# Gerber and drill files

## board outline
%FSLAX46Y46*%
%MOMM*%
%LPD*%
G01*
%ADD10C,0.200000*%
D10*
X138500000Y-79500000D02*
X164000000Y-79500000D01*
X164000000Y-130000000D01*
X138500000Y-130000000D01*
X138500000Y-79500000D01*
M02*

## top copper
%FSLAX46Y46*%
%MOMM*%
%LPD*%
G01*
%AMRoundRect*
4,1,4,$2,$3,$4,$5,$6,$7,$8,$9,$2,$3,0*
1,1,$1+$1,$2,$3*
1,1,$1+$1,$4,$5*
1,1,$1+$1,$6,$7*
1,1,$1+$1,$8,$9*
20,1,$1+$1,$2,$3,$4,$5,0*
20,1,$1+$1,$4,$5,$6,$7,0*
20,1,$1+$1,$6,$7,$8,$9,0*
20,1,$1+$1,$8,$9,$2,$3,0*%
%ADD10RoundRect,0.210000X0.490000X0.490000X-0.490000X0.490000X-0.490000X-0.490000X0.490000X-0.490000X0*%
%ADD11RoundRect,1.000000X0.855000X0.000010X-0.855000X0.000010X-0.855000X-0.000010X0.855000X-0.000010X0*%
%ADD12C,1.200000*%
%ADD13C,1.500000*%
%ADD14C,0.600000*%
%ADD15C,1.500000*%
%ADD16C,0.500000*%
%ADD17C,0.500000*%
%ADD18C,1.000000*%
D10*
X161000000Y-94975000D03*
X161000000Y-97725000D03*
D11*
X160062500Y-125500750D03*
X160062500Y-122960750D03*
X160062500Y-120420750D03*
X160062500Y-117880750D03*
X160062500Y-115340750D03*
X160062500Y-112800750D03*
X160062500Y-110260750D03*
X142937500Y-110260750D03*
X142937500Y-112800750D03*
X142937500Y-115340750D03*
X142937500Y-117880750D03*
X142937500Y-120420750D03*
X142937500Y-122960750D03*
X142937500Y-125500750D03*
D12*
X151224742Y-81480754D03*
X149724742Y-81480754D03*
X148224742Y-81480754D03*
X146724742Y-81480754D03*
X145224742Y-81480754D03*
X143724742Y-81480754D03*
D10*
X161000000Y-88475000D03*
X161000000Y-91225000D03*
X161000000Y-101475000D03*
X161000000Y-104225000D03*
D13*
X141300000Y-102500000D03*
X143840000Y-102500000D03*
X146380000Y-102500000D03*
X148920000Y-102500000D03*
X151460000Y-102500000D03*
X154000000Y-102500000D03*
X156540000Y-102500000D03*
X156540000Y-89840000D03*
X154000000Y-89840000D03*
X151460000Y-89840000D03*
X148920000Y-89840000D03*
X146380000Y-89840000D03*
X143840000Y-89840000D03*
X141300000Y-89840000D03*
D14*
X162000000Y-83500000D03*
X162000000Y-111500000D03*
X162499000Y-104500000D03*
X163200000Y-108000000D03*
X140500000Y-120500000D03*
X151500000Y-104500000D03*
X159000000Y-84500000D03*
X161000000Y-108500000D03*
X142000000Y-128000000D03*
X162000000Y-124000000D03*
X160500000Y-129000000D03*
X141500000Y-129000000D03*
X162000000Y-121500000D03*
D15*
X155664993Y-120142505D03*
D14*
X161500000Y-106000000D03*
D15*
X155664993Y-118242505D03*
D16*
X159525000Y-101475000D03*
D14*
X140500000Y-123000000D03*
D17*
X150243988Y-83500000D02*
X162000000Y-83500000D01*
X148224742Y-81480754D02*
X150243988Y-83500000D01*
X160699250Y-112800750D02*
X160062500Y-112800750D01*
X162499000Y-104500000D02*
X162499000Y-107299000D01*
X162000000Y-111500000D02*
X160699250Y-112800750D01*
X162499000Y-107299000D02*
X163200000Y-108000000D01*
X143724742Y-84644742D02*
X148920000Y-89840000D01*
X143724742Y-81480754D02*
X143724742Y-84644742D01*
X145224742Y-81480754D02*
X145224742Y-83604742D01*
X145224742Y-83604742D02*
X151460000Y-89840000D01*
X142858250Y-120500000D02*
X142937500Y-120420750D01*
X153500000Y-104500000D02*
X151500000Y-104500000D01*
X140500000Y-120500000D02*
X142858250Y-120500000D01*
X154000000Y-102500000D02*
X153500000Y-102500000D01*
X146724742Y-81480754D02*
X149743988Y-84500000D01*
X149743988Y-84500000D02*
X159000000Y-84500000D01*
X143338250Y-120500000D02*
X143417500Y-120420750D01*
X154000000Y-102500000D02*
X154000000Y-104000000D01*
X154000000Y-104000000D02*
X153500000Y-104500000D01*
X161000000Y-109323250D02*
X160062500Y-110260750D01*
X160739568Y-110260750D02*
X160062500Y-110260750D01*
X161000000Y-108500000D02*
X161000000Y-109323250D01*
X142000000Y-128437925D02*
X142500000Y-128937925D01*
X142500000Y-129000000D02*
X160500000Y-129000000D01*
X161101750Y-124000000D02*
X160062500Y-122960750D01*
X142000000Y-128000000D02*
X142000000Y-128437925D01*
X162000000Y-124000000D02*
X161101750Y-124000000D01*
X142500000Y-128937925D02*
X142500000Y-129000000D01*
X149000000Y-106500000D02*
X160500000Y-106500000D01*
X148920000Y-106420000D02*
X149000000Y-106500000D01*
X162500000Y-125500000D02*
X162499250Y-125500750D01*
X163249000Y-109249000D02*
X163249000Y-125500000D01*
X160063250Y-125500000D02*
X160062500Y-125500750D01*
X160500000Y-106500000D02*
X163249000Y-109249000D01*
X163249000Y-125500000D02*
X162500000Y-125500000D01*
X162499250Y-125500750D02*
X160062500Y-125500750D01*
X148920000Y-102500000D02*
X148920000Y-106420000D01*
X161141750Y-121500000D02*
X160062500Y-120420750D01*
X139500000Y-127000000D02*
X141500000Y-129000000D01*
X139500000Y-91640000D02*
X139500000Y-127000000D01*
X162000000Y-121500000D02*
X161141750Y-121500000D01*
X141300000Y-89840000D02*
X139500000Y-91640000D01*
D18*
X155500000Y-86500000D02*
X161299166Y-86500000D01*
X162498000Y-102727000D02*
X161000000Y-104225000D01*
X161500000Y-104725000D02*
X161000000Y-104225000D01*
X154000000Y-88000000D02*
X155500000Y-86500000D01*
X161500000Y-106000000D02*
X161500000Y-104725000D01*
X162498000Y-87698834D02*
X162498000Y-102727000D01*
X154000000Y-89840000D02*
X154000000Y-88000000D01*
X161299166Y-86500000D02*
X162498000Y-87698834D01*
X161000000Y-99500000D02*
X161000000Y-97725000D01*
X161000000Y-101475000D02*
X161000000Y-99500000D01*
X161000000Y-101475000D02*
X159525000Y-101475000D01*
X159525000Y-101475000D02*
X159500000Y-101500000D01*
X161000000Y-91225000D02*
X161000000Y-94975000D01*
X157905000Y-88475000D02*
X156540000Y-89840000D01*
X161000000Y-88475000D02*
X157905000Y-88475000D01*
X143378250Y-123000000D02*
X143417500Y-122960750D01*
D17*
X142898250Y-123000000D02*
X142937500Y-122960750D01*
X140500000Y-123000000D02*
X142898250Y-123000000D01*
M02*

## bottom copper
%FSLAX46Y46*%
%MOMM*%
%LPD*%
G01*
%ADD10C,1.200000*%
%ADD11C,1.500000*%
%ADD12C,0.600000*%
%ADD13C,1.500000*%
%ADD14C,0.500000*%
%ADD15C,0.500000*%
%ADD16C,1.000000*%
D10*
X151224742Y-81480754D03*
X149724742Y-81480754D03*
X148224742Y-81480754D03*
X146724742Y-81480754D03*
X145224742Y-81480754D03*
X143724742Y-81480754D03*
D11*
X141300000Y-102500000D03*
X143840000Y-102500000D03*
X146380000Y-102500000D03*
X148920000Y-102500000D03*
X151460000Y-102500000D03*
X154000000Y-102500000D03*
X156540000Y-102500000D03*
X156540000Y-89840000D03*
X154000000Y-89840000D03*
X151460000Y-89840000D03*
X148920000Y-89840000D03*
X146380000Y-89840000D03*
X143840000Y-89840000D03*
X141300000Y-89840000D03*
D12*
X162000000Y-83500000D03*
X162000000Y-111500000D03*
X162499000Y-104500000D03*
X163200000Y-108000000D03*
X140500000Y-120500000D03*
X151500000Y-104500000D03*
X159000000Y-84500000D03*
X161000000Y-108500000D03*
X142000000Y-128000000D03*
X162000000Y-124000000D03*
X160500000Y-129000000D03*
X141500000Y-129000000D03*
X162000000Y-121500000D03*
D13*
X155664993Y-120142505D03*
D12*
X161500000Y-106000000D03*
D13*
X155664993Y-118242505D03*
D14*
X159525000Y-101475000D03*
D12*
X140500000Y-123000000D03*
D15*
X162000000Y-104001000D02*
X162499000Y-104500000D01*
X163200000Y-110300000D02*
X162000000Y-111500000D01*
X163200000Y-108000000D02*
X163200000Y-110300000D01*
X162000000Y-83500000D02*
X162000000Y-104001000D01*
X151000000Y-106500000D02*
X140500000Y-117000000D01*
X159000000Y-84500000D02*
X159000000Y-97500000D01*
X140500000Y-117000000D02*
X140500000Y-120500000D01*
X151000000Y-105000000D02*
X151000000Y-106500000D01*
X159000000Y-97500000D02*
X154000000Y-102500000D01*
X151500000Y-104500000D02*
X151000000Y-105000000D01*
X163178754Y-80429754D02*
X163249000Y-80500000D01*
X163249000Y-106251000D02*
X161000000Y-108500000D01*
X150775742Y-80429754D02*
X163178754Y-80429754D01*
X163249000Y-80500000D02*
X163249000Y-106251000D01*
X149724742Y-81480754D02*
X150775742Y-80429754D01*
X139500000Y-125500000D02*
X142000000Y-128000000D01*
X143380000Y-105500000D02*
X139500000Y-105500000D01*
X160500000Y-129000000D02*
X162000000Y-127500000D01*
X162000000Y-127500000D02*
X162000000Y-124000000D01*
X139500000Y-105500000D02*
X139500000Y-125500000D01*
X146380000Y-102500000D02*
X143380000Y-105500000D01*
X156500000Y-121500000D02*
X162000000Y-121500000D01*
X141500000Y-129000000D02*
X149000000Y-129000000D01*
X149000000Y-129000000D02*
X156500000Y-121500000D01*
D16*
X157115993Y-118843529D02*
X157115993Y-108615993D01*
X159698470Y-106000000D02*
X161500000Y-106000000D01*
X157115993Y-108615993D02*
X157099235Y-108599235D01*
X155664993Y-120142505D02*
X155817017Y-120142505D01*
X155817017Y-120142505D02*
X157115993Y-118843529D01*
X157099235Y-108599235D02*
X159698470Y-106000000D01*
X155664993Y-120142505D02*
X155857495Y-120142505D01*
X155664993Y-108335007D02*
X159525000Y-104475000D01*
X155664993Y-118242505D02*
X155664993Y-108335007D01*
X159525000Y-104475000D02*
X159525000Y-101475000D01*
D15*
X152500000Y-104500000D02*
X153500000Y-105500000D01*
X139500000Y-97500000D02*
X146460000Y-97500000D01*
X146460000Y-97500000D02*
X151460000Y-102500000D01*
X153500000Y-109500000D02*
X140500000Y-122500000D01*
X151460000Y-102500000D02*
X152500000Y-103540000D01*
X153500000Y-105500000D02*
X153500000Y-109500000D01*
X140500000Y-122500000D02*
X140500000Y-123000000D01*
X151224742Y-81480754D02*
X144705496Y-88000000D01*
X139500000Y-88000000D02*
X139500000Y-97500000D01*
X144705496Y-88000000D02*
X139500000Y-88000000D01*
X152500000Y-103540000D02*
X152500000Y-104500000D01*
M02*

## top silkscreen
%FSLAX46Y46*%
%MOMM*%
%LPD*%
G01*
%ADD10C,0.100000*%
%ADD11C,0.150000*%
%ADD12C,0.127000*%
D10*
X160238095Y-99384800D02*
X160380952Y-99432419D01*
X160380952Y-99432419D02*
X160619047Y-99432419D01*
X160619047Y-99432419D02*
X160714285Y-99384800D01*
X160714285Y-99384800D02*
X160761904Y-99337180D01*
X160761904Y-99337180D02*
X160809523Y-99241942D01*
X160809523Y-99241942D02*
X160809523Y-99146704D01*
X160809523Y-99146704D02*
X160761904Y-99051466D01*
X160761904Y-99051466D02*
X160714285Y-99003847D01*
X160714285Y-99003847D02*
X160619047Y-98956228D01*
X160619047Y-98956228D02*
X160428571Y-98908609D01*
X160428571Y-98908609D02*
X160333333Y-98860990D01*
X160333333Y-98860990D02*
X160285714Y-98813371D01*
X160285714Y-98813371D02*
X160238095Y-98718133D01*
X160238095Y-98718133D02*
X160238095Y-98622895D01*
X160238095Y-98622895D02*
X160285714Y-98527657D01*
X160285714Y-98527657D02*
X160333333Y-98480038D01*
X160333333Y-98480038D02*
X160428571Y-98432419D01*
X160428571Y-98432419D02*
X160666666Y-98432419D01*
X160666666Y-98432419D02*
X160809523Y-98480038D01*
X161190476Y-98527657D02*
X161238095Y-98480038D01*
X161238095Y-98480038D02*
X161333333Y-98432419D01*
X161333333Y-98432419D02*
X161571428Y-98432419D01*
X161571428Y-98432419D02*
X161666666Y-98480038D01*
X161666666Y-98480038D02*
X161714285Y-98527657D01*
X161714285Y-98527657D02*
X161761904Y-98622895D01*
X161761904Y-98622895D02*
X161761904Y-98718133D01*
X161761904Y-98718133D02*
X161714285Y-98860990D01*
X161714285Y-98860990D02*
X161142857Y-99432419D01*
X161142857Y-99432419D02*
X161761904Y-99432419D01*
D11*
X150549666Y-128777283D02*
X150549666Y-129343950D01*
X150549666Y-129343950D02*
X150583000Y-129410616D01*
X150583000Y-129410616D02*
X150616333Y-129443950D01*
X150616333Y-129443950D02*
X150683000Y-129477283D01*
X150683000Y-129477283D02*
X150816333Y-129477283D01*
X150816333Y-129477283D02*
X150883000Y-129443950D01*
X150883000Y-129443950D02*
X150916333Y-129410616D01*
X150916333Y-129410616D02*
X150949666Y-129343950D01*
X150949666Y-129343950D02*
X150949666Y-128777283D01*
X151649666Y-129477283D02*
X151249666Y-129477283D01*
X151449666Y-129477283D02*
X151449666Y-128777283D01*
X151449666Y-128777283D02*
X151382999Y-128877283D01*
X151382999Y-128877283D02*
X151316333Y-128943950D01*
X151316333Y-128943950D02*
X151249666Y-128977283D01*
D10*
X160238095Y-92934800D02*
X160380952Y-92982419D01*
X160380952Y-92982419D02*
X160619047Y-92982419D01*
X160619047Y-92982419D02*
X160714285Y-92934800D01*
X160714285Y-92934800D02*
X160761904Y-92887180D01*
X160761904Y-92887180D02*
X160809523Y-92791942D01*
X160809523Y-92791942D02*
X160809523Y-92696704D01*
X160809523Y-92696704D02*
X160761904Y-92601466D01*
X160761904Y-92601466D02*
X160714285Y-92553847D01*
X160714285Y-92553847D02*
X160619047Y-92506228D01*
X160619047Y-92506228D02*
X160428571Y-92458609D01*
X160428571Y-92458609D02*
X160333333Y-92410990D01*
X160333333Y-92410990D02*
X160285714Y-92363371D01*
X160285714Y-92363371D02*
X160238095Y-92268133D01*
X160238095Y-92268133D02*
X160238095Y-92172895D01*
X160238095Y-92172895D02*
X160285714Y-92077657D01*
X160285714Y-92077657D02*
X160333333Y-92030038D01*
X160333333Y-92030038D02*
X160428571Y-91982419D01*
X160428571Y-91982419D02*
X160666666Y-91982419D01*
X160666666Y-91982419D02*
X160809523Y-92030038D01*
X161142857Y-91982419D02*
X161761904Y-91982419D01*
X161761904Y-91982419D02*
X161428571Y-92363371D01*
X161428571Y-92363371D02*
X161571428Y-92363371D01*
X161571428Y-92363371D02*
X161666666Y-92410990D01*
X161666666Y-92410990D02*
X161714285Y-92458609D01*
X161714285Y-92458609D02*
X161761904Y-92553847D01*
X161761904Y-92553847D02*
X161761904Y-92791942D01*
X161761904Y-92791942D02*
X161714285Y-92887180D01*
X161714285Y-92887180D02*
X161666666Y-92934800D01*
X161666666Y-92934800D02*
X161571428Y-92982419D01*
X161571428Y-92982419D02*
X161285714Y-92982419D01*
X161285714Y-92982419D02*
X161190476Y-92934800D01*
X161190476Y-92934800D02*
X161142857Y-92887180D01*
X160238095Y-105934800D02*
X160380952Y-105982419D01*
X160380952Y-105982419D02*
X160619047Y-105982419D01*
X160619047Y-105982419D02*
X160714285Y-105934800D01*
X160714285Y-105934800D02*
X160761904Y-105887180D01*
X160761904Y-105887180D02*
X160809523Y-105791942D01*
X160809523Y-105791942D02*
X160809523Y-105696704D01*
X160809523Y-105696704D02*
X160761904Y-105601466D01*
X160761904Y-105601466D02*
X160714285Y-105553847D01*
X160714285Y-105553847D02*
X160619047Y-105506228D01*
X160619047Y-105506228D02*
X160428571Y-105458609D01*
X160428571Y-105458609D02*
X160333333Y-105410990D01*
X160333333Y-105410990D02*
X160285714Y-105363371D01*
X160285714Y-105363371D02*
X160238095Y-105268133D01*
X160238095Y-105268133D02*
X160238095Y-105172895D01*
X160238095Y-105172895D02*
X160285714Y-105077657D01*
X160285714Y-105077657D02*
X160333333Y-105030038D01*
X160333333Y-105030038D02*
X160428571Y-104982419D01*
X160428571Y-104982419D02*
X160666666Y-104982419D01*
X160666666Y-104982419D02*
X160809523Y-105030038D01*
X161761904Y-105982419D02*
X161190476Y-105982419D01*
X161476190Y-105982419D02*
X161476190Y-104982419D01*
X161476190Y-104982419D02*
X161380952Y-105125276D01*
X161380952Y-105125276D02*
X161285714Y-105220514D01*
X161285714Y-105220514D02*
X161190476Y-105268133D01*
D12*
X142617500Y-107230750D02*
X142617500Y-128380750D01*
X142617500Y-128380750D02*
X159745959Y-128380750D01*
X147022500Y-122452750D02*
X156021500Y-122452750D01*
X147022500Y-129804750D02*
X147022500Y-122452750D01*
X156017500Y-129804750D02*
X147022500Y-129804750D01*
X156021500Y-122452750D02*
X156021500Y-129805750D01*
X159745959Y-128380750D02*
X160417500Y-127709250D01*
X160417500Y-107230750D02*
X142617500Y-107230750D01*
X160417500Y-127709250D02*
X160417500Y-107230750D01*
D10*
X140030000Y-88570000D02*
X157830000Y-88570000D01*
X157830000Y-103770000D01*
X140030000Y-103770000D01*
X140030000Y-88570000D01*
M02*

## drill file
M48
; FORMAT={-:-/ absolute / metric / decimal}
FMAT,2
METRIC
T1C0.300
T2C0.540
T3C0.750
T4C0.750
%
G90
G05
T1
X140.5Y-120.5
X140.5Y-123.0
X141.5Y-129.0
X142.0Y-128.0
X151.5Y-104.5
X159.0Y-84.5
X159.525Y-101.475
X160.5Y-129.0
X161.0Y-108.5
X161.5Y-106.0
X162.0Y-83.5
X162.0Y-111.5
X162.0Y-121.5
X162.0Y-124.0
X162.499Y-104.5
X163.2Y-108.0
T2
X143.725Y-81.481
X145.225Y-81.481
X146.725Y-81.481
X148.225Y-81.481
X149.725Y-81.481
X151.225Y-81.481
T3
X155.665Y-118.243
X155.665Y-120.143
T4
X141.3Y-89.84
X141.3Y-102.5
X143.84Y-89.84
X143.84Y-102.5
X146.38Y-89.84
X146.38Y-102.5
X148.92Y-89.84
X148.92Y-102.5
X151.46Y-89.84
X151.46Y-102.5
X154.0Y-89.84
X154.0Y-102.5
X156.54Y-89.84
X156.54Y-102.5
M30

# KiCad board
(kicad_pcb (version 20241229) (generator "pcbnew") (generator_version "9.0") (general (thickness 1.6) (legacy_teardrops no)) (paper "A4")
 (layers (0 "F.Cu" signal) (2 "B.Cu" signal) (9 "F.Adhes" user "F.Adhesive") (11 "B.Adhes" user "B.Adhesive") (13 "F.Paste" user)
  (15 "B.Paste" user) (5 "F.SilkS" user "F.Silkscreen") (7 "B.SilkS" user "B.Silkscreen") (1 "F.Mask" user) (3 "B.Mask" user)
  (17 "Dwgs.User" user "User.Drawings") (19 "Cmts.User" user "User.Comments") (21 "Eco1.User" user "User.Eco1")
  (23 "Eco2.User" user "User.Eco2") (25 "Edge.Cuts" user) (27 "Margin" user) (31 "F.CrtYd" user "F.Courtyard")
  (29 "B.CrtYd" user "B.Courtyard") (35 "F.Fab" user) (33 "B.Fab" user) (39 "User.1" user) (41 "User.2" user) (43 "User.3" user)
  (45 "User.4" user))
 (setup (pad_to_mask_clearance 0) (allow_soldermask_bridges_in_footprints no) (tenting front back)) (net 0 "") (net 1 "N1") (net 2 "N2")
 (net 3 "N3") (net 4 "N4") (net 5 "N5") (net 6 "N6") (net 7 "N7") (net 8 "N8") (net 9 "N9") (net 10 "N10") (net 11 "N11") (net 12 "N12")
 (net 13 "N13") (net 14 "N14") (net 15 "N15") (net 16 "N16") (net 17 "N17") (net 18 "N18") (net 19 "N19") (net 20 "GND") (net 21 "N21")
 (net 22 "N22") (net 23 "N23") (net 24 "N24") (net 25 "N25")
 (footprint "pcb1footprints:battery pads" (layer "F.Cu") (at 161 101.475 180)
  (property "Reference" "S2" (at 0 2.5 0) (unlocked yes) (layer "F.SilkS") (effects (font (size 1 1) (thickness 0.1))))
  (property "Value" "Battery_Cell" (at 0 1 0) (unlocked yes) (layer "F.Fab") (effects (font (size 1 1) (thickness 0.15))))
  (pad "1" smd roundrect (at 0 6.5 180) (size 1.4 1.4) (layers "F.Cu" "F.Mask" "F.Paste") (roundrect_rratio 0.15) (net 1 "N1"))
  (pad "2" smd roundrect (at 0 3.75 180) (size 1.4 1.4) (layers "F.Cu" "F.Mask" "F.Paste") (roundrect_rratio 0.15) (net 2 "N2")))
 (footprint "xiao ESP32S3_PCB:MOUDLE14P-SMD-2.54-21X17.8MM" (layer "F.Cu") (at 160.4175 107.38075 180)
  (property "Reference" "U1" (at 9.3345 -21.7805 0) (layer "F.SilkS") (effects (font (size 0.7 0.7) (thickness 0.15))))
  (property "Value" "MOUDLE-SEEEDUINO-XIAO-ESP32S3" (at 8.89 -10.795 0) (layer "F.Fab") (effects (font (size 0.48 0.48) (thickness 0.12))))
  (fp_line (start 17.8 0.15) (end 17.8 -21) (stroke (width 0.127) (type solid)) (layer "F.SilkS"))
  (fp_line (start 17.8 -21) (end 0.671541 -21) (stroke (width 0.127) (type solid)) (layer "F.SilkS"))
  (fp_line (start 13.395 -15.072) (end 4.396 -15.072) (stroke (width 0.127) (type solid)) (layer "F.SilkS"))
  (fp_line (start 13.395 -22.424) (end 13.395 -15.072) (stroke (width 0.127) (type solid)) (layer "F.SilkS"))
  (fp_line (start 4.4 -22.424) (end 13.395 -22.424) (stroke (width 0.127) (type solid)) (layer "F.SilkS"))
  (fp_line (start 4.396 -15.072) (end 4.396 -22.425) (stroke (width 0.127) (type solid)) (layer "F.SilkS"))
  (fp_line (start 0.671541 -21) (end 0 -20.3285) (stroke (width 0.127) (type solid)) (layer "F.SilkS"))
  (fp_line (start 0 0.15) (end 17.8 0.15) (stroke (width 0.127) (type solid)) (layer "F.SilkS"))
  (fp_line (start 0 -20.3285) (end 0 0.15) (stroke (width 0.127) (type solid)) (layer "F.SilkS"))
  (pad "1" smd roundrect (at 0.355 -18.12 180) (size 3.71 2) (layers "F.Cu" "F.Mask" "F.Paste") (roundrect_rratio 0.5) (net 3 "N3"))
  (pad "2" smd roundrect (at 0.355 -15.58 180) (size 3.71 2) (layers "F.Cu" "F.Mask" "F.Paste") (roundrect_rratio 0.5) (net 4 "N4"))
  (pad "3" smd roundrect (at 0.355 -13.04 180) (size 3.71 2) (layers "F.Cu" "F.Mask" "F.Paste") (roundrect_rratio 0.5) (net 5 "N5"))
  (pad "4" smd roundrect (at 0.355 -10.5 180) (size 3.71 2) (layers "F.Cu" "F.Mask" "F.Paste") (roundrect_rratio 0.5) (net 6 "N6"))
  (pad "5" smd roundrect (at 0.355 -7.96 180) (size 3.71 2) (layers "F.Cu" "F.Mask" "F.Paste") (roundrect_rratio 0.5) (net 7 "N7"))
  (pad "6" smd roundrect (at 0.355 -5.42 180) (size 3.71 2) (layers "F.Cu" "F.Mask" "F.Paste") (roundrect_rratio 0.5) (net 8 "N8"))
  (pad "7" smd roundrect (at 0.355 -2.88 180) (size 3.71 2) (layers "F.Cu" "F.Mask" "F.Paste") (roundrect_rratio 0.5) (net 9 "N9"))
  (pad "8" smd roundrect (at 17.48 -2.88 180) (size 3.71 2) (layers "F.Cu" "F.Mask" "F.Paste") (roundrect_rratio 0.5) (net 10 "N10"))
  (pad "9" smd roundrect (at 17.48 -5.42 180) (size 3.71 2) (layers "F.Cu" "F.Mask" "F.Paste") (roundrect_rratio 0.5) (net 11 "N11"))
  (pad "10" smd roundrect (at 17.48 -7.96 180) (size 3.71 2) (layers "F.Cu" "F.Mask" "F.Paste") (roundrect_rratio 0.5) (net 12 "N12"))
  (pad "11" smd roundrect (at 17.48 -10.5 180) (size 3.71 2) (layers "F.Cu" "F.Mask" "F.Paste") (roundrect_rratio 0.5) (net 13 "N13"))
  (pad "12" smd roundrect (at 17.48 -13.04 180) (size 3.71 2) (layers "F.Cu" "F.Mask" "F.Paste") (roundrect_rratio 0.5) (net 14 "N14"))
  (pad "13" smd roundrect (at 17.48 -15.58 180) (size 3.71 2) (layers "F.Cu" "F.Mask" "F.Paste") (roundrect_rratio 0.5) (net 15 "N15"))
  (pad "14" smd roundrect (at 17.48 -18.12 180) (size 3.71 2) (layers "F.Cu" "F.Mask" "F.Paste") (roundrect_rratio 0.5) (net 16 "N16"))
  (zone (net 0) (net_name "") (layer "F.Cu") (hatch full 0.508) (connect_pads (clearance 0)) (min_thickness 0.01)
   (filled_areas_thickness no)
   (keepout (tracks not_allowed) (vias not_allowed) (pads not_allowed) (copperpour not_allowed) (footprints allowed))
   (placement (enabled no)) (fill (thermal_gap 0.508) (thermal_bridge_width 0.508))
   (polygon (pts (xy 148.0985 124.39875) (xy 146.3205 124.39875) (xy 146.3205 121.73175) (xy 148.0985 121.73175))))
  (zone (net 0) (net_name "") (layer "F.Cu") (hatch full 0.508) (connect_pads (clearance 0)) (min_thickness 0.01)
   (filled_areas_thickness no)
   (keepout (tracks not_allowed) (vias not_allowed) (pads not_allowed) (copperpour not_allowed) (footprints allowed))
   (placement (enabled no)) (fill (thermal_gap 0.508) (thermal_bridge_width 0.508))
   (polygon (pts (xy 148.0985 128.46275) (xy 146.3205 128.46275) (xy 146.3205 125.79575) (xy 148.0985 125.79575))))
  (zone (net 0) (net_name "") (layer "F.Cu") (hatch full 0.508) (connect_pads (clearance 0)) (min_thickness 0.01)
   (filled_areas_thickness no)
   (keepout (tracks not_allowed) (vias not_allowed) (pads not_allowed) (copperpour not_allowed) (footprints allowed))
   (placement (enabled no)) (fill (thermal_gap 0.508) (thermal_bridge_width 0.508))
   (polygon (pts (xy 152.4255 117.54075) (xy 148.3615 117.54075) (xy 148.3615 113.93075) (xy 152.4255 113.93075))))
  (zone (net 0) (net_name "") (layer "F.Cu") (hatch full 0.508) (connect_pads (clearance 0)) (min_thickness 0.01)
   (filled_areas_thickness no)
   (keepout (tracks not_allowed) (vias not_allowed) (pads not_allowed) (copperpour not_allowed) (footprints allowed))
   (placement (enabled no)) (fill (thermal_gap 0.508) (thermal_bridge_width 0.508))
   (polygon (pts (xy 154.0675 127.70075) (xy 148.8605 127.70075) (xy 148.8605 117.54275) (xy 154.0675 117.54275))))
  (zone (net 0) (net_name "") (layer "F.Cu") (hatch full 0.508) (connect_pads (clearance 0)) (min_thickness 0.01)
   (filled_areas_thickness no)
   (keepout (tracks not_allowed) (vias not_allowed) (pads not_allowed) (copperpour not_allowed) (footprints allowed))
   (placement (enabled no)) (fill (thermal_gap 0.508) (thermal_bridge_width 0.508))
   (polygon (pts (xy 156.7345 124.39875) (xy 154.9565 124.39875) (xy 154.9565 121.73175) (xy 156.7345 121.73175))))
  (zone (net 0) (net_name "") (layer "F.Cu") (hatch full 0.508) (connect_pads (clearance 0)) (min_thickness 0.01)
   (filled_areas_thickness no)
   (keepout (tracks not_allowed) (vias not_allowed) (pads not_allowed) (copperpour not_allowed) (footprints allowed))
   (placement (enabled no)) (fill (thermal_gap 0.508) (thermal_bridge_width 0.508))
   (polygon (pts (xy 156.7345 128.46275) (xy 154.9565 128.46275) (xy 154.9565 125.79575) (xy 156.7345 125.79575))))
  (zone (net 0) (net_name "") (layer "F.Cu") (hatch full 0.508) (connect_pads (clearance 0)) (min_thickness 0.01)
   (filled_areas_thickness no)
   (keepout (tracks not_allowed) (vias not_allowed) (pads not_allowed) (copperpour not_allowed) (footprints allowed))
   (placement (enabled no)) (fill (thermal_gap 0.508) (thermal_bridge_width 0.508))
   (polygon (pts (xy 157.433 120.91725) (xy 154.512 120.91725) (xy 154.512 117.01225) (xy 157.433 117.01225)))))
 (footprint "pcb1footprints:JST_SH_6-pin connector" (layer "F.Cu") (at 147.5 81.5 180)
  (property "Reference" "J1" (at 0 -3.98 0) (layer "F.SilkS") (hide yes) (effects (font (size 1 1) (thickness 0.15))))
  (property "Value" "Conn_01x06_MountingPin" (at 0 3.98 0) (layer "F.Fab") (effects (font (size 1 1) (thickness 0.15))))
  (pad "1" thru_hole circle (at -3.724742 0.019246 180) (size 1.2 1.2) (drill 0.54) (layers "*.Cu" "*.Mask") (remove_unused_layers no)
   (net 15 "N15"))
  (pad "2" thru_hole circle (at -2.224742 0.019246 180) (size 1.2 1.2) (drill 0.54) (layers "*.Cu" "*.Mask") (remove_unused_layers no)
   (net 9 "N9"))
  (pad "3" thru_hole circle (at -0.724742 0.019246 180) (size 1.2 1.2) (drill 0.54) (layers "*.Cu" "*.Mask") (remove_unused_layers no)
   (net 8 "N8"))
  (pad "4" thru_hole circle (at 0.775258 0.019246 180) (size 1.2 1.2) (drill 0.54) (layers "*.Cu" "*.Mask") (remove_unused_layers no)
   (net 14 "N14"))
  (pad "5" thru_hole circle (at 2.275258 0.019246 180) (size 1.2 1.2) (drill 0.54) (layers "*.Cu" "*.Mask") (remove_unused_layers no)
   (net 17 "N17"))
  (pad "6" thru_hole circle (at 3.775258 0.019246 180) (size 1.2 1.2) (drill 0.54) (layers "*.Cu" "*.Mask") (remove_unused_layers no)
   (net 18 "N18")))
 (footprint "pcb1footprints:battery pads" (layer "F.Cu") (at 161 94.975 180)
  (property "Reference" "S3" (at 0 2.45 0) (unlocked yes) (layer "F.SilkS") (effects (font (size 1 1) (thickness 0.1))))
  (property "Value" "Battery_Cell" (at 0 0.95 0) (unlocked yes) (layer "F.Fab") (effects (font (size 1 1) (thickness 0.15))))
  (pad "1" smd roundrect (at 0 6.5 180) (size 1.4 1.4) (layers "F.Cu" "F.Mask" "F.Paste") (roundrect_rratio 0.15) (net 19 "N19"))
  (pad "2" smd roundrect (at 0 3.75 180) (size 1.4 1.4) (layers "F.Cu" "F.Mask" "F.Paste") (roundrect_rratio 0.15) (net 1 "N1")))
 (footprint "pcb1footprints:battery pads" (layer "F.Cu") (at 161 107.975 180)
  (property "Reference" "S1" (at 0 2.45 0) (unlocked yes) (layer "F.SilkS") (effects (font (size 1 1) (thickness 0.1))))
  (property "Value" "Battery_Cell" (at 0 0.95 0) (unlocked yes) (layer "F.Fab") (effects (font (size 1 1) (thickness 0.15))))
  (pad "1" smd roundrect (at 0 6.5 180) (size 1.4 1.4) (layers "F.Cu" "F.Mask" "F.Paste") (roundrect_rratio 0.15) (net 2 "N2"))
  (pad "2" smd roundrect (at 0 3.75 180) (size 1.4 1.4) (layers "F.Cu" "F.Mask" "F.Paste") (roundrect_rratio 0.15) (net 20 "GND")))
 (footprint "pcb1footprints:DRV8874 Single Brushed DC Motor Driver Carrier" (layer "F.Cu") (at 148.93 96.17 90)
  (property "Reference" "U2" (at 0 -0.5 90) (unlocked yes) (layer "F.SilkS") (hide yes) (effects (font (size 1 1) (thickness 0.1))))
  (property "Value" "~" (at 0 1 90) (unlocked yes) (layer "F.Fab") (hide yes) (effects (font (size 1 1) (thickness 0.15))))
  (fp_rect (start -7.6 -8.9) (end 7.6 8.9) (stroke (width 0.1) (type solid)) (fill no) (layer "F.SilkS"))
  (pad "1" thru_hole circle (at -6.33 -7.63 90) (size 1.5 1.5) (drill 0.75) (layers "*.Cu" "*.Mask") (remove_unused_layers no)
   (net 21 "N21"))
  (pad "2" thru_hole circle (at -6.33 -5.09 90) (size 1.5 1.5) (drill 0.75) (layers "*.Cu" "*.Mask") (remove_unused_layers no)
   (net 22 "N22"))
  (pad "3" thru_hole circle (at -6.33 -2.55 90) (size 1.5 1.5) (drill 0.75) (layers "*.Cu" "*.Mask") (remove_unused_layers no) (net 4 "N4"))
  (pad "4" thru_hole circle (at -6.33 -0.01 90) (size 1.5 1.5) (drill 0.75) (layers "*.Cu" "*.Mask") (remove_unused_layers no) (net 3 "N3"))
  (pad "5" thru_hole circle (at -6.33 2.53 90) (size 1.5 1.5) (drill 0.75) (layers "*.Cu" "*.Mask") (remove_unused_layers no) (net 15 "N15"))
  (pad "6" thru_hole circle (at -6.33 5.07 90) (size 1.5 1.5) (drill 0.75) (layers "*.Cu" "*.Mask") (remove_unused_layers no) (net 14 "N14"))
  (pad "7" thru_hole circle (at -6.33 7.61 90) (size 1.5 1.5) (drill 0.75) (layers "*.Cu" "*.Mask") (remove_unused_layers no) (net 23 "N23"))
  (pad "8" thru_hole circle (at 6.33 7.61 90) (size 1.5 1.5) (drill 0.75) (layers "*.Cu" "*.Mask") (remove_unused_layers no) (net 19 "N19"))
  (pad "9" thru_hole circle (at 6.33 5.07 90) (size 1.5 1.5) (drill 0.75) (layers "*.Cu" "*.Mask") (remove_unused_layers no) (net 20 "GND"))
  (pad "10" thru_hole circle (at 6.33 2.53 90) (size 1.5 1.5) (drill 0.75) (layers "*.Cu" "*.Mask") (remove_unused_layers no) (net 17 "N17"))
  (pad "11" thru_hole circle (at 6.33 -0.01 90) (size 1.5 1.5) (drill 0.75) (layers "*.Cu" "*.Mask") (remove_unused_layers no)
   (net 18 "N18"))
  (pad "12" thru_hole circle (at 6.33 -2.55 90) (size 1.5 1.5) (drill 0.75) (layers "*.Cu" "*.Mask") (remove_unused_layers no)
   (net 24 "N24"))
  (pad "13" thru_hole circle (at 6.33 -5.09 90) (size 1.5 1.5) (drill 0.75) (layers "*.Cu" "*.Mask") (remove_unused_layers no)
   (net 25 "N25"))
  (pad "14" thru_hole circle (at 6.33 -7.63 90) (size 1.5 1.5) (drill 0.75) (layers "*.Cu" "*.Mask") (remove_unused_layers no) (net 5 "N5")))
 (gr_rect (start 138.5 79.5) (end 164 130) (stroke (width 0.2) (type solid)) (fill no) (layer "Edge.Cuts"))
 (segment (start 150.243988 83.5) (end 162 83.5) (width 0.5) (layer "F.Cu") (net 8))
 (segment (start 148.224742 81.480754) (end 150.243988 83.5) (width 0.5) (layer "F.Cu") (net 8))
 (segment (start 160.69925 112.80075) (end 160.0625 112.80075) (width 0.5) (layer "F.Cu") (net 8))
 (segment (start 162.499 104.5) (end 162.499 107.299) (width 0.5) (layer "F.Cu") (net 8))
 (segment (start 162 111.5) (end 160.69925 112.80075) (width 0.5) (layer "F.Cu") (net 8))
 (segment (start 162.499 107.299) (end 163.2 108) (width 0.5) (layer "F.Cu") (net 8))
 (via (at 162 83.5) (size 0.6) (drill 0.3) (layers "F.Cu" "B.Cu") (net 8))
 (via (at 162 111.5) (size 0.6) (drill 0.3) (layers "F.Cu" "B.Cu") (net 8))
 (via (at 162.499 104.5) (size 0.6) (drill 0.3) (layers "F.Cu" "B.Cu") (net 8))
 (via (at 163.2 108) (size 0.6) (drill 0.3) (layers "F.Cu" "B.Cu") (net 8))
 (segment (start 162 104.001) (end 162.499 104.5) (width 0.5) (layer "B.Cu") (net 8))
 (segment (start 163.2 110.3) (end 162 111.5) (width 0.5) (layer "B.Cu") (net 8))
 (segment (start 163.2 108) (end 163.2 110.3) (width 0.5) (layer "B.Cu") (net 8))
 (segment (start 162 83.5) (end 162 104.001) (width 0.5) (layer "B.Cu") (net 8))
 (segment (start 143.724742 84.644742) (end 148.92 89.84) (width 0.5) (layer "F.Cu") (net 18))
 (segment (start 143.724742 81.480754) (end 143.724742 84.644742) (width 0.5) (layer "F.Cu") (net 18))
 (segment (start 145.224742 81.480754) (end 145.224742 83.604742) (width 0.5) (layer "F.Cu") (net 17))
 (segment (start 145.224742 83.604742) (end 151.46 89.84) (width 0.5) (layer "F.Cu") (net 17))
 (segment (start 142.85825 120.5) (end 142.9375 120.42075) (width 0.5) (layer "F.Cu") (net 14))
 (segment (start 153.5 104.5) (end 151.5 104.5) (width 0.5) (layer "F.Cu") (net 14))
 (segment (start 140.5 120.5) (end 142.85825 120.5) (width 0.5) (layer "F.Cu") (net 14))
 (segment (start 154 102.5) (end 153.5 102.5) (width 0.5) (layer "F.Cu") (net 14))
 (segment (start 146.724742 81.480754) (end 149.743988 84.5) (width 0.5) (layer "F.Cu") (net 14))
 (segment (start 149.743988 84.5) (end 159 84.5) (width 0.5) (layer "F.Cu") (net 14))
 (segment (start 143.33825 120.5) (end 143.4175 120.42075) (width 0.5) (layer "F.Cu") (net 14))
 (segment (start 154 102.5) (end 154 104) (width 0.5) (layer "F.Cu") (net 14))
 (segment (start 154 104) (end 153.5 104.5) (width 0.5) (layer "F.Cu") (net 14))
 (via (at 140.5 120.5) (size 0.6) (drill 0.3) (layers "F.Cu" "B.Cu") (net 14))
 (via (at 151.5 104.5) (size 0.6) (drill 0.3) (layers "F.Cu" "B.Cu") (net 14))
 (via (at 159 84.5) (size 0.6) (drill 0.3) (layers "F.Cu" "B.Cu") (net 14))
 (segment (start 151 106.5) (end 140.5 117) (width 0.5) (layer "B.Cu") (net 14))
 (segment (start 159 84.5) (end 159 97.5) (width 0.5) (layer "B.Cu") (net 14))
 (segment (start 140.5 117) (end 140.5 120.5) (width 0.5) (layer "B.Cu") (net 14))
 (segment (start 151 105) (end 151 106.5) (width 0.5) (layer "B.Cu") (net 14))
 (segment (start 159 97.5) (end 154 102.5) (width 0.5) (layer "B.Cu") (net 14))
 (segment (start 151.5 104.5) (end 151 105) (width 0.5) (layer "B.Cu") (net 14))
 (segment (start 161 109.32325) (end 160.0625 110.26075) (width 0.5) (layer "F.Cu") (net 9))
 (segment (start 160.739568 110.26075) (end 160.0625 110.26075) (width 0.5) (layer "F.Cu") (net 9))
 (segment (start 161 108.5) (end 161 109.32325) (width 0.5) (layer "F.Cu") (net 9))
 (via (at 161 108.5) (size 0.6) (drill 0.3) (layers "F.Cu" "B.Cu") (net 9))
 (segment (start 163.178754 80.429754) (end 163.249 80.5) (width 0.5) (layer "B.Cu") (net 9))
 (segment (start 163.249 106.251) (end 161 108.5) (width 0.5) (layer "B.Cu") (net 9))
 (segment (start 150.775742 80.429754) (end 163.178754 80.429754) (width 0.5) (layer "B.Cu") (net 9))
 (segment (start 163.249 80.5) (end 163.249 106.251) (width 0.5) (layer "B.Cu") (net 9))
 (segment (start 149.724742 81.480754) (end 150.775742 80.429754) (width 0.5) (layer "B.Cu") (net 9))
 (segment (start 142 128.437925) (end 142.5 128.937925) (width 0.5) (layer "F.Cu") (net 4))
 (segment (start 142.5 129) (end 160.5 129) (width 0.5) (layer "F.Cu") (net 4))
 (segment (start 161.10175 124) (end 160.0625 122.96075) (width 0.5) (layer "F.Cu") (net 4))
 (segment (start 142 128) (end 142 128.437925) (width 0.5) (layer "F.Cu") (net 4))
 (segment (start 162 124) (end 161.10175 124) (width 0.5) (layer "F.Cu") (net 4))
 (segment (start 142.5 128.937925) (end 142.5 129) (width 0.5) (layer "F.Cu") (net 4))
 (via (at 142 128) (size 0.6) (drill 0.3) (layers "F.Cu" "B.Cu") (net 4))
 (via (at 162 124) (size 0.6) (drill 0.3) (layers "F.Cu" "B.Cu") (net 4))
 (via (at 160.5 129) (size 0.6) (drill 0.3) (layers "F.Cu" "B.Cu") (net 4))
 (segment (start 139.5 125.5) (end 142 128) (width 0.5) (layer "B.Cu") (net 4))
 (segment (start 143.38 105.5) (end 139.5 105.5) (width 0.5) (layer "B.Cu") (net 4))
 (segment (start 160.5 129) (end 162 127.5) (width 0.5) (layer "B.Cu") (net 4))
 (segment (start 162 127.5) (end 162 124) (width 0.5) (layer "B.Cu") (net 4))
 (segment (start 139.5 105.5) (end 139.5 125.5) (width 0.5) (layer "B.Cu") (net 4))
 (segment (start 146.38 102.5) (end 143.38 105.5) (width 0.5) (layer "B.Cu") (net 4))
 (segment (start 149 106.5) (end 160.5 106.5) (width 0.5) (layer "F.Cu") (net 3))
 (segment (start 148.92 106.42) (end 149 106.5) (width 0.5) (layer "F.Cu") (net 3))
 (segment (start 162.5 125.5) (end 162.49925 125.50075) (width 0.5) (layer "F.Cu") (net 3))
 (segment (start 163.249 109.249) (end 163.249 125.5) (width 0.5) (layer "F.Cu") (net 3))
 (segment (start 160.06325 125.5) (end 160.0625 125.50075) (width 0.5) (layer "F.Cu") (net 3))
 (segment (start 160.5 106.5) (end 163.249 109.249) (width 0.5) (layer "F.Cu") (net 3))
 (segment (start 163.249 125.5) (end 162.5 125.5) (width 0.5) (layer "F.Cu") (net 3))
 (segment (start 162.49925 125.50075) (end 160.0625 125.50075) (width 0.5) (layer "F.Cu") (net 3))
 (segment (start 148.92 102.5) (end 148.92 106.42) (width 0.5) (layer "F.Cu") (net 3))
 (segment (start 161.14175 121.5) (end 160.0625 120.42075) (width 0.5) (layer "F.Cu") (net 5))
 (segment (start 139.5 127) (end 141.5 129) (width 0.5) (layer "F.Cu") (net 5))
 (segment (start 139.5 91.64) (end 139.5 127) (width 0.5) (layer "F.Cu") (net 5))
 (segment (start 162 121.5) (end 161.14175 121.5) (width 0.5) (layer "F.Cu") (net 5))
 (segment (start 141.3 89.84) (end 139.5 91.64) (width 0.5) (layer "F.Cu") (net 5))
 (via (at 141.5 129) (size 0.6) (drill 0.3) (layers "F.Cu" "B.Cu") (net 5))
 (via (at 162 121.5) (size 0.6) (drill 0.3) (layers "F.Cu" "B.Cu") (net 5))
 (segment (start 156.5 121.5) (end 162 121.5) (width 0.5) (layer "B.Cu") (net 5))
 (segment (start 141.5 129) (end 149 129) (width 0.5) (layer "B.Cu") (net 5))
 (segment (start 149 129) (end 156.5 121.5) (width 0.5) (layer "B.Cu") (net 5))
 (segment (start 155.5 86.5) (end 161.299166 86.5) (width 1) (layer "F.Cu") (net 20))
 (segment (start 162.498 102.727) (end 161 104.225) (width 1) (layer "F.Cu") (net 20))
 (segment (start 161.5 104.725) (end 161 104.225) (width 1) (layer "F.Cu") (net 20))
 (segment (start 154 88) (end 155.5 86.5) (width 1) (layer "F.Cu") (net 20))
 (segment (start 161.5 106) (end 161.5 104.725) (width 1) (layer "F.Cu") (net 20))
 (segment (start 162.498 87.698834) (end 162.498 102.727) (width 1) (layer "F.Cu") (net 20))
 (segment (start 154 89.84) (end 154 88) (width 1) (layer "F.Cu") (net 20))
 (segment (start 161.299166 86.5) (end 162.498 87.698834) (width 1) (layer "F.Cu") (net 20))
 (via (at 155.664993 120.142505) (size 1.5) (drill 0.75) (layers "F.Cu" "B.Cu") (tenting none) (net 20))
 (via (at 161.5 106) (size 0.6) (drill 0.3) (layers "F.Cu" "B.Cu") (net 20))
 (segment (start 157.115993 118.843529) (end 157.115993 108.615993) (width 1) (layer "B.Cu") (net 20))
 (segment (start 159.69847 106) (end 161.5 106) (width 1) (layer "B.Cu") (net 20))
 (segment (start 157.115993 108.615993) (end 157.099235 108.599235) (width 1) (layer "B.Cu") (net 20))
 (segment (start 155.664993 120.142505) (end 155.817017 120.142505) (width 1) (layer "B.Cu") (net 20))
 (segment (start 155.817017 120.142505) (end 157.115993 118.843529) (width 1) (layer "B.Cu") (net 20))
 (segment (start 157.099235 108.599235) (end 159.69847 106) (width 1) (layer "B.Cu") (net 20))
 (segment (start 155.664993 120.142505) (end 155.857495 120.142505) (width 1) (layer "B.Cu") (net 20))
 (segment (start 161 99.5) (end 161 97.725) (width 1) (layer "F.Cu") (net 2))
 (segment (start 161 101.475) (end 161 99.5) (width 1) (layer "F.Cu") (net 2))
 (segment (start 161 101.475) (end 159.525 101.475) (width 1) (layer "F.Cu") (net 2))
 (segment (start 159.525 101.475) (end 159.5 101.5) (width 1) (layer "F.Cu") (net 2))
 (via (at 155.664993 118.242505) (size 1.5) (drill 0.75) (layers "F.Cu" "B.Cu") (tenting none) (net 2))
 (via (at 159.525 101.475) (size 0.5) (drill 0.3) (layers "F.Cu" "B.Cu") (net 2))
 (segment (start 155.664993 108.335007) (end 159.525 104.475) (width 1) (layer "B.Cu") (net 2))
 (segment (start 155.664993 118.242505) (end 155.664993 108.335007) (width 1) (layer "B.Cu") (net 2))
 (segment (start 159.525 104.475) (end 159.525 101.475) (width 1) (layer "B.Cu") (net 2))
 (segment (start 161 91.225) (end 161 94.975) (width 1) (layer "F.Cu") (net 1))
 (segment (start 157.905 88.475) (end 156.54 89.84) (width 1) (layer "F.Cu") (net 19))
 (segment (start 161 88.475) (end 157.905 88.475) (width 1) (layer "F.Cu") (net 19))
 (segment (start 143.37825 123) (end 143.4175 122.96075) (width 1) (layer "F.Cu") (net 15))
 (segment (start 142.89825 123) (end 142.9375 122.96075) (width 0.5) (layer "F.Cu") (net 15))
 (segment (start 140.5 123) (end 142.89825 123) (width 0.5) (layer "F.Cu") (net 15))
 (via (at 140.5 123) (size 0.6) (drill 0.3) (layers "F.Cu" "B.Cu") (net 15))
 (segment (start 152.5 104.5) (end 153.5 105.5) (width 0.5) (layer "B.Cu") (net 15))
 (segment (start 139.5 97.5) (end 146.46 97.5) (width 0.5) (layer "B.Cu") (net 15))
 (segment (start 146.46 97.5) (end 151.46 102.5) (width 0.5) (layer "B.Cu") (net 15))
 (segment (start 153.5 109.5) (end 140.5 122.5) (width 0.5) (layer "B.Cu") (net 15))
 (segment (start 151.46 102.5) (end 152.5 103.54) (width 0.5) (layer "B.Cu") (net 15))
 (segment (start 153.5 105.5) (end 153.5 109.5) (width 0.5) (layer "B.Cu") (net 15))
 (segment (start 140.5 122.5) (end 140.5 123) (width 0.5) (layer "B.Cu") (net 15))
 (segment (start 151.224742 81.480754) (end 144.705496 88) (width 0.5) (layer "B.Cu") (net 15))
 (segment (start 139.5 88) (end 139.5 97.5) (width 0.5) (layer "B.Cu") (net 15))
 (segment (start 144.705496 88) (end 139.5 88) (width 0.5) (layer "B.Cu") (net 15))
 (segment (start 152.5 103.54) (end 152.5 104.5) (width 0.5) (layer "B.Cu") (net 15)))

